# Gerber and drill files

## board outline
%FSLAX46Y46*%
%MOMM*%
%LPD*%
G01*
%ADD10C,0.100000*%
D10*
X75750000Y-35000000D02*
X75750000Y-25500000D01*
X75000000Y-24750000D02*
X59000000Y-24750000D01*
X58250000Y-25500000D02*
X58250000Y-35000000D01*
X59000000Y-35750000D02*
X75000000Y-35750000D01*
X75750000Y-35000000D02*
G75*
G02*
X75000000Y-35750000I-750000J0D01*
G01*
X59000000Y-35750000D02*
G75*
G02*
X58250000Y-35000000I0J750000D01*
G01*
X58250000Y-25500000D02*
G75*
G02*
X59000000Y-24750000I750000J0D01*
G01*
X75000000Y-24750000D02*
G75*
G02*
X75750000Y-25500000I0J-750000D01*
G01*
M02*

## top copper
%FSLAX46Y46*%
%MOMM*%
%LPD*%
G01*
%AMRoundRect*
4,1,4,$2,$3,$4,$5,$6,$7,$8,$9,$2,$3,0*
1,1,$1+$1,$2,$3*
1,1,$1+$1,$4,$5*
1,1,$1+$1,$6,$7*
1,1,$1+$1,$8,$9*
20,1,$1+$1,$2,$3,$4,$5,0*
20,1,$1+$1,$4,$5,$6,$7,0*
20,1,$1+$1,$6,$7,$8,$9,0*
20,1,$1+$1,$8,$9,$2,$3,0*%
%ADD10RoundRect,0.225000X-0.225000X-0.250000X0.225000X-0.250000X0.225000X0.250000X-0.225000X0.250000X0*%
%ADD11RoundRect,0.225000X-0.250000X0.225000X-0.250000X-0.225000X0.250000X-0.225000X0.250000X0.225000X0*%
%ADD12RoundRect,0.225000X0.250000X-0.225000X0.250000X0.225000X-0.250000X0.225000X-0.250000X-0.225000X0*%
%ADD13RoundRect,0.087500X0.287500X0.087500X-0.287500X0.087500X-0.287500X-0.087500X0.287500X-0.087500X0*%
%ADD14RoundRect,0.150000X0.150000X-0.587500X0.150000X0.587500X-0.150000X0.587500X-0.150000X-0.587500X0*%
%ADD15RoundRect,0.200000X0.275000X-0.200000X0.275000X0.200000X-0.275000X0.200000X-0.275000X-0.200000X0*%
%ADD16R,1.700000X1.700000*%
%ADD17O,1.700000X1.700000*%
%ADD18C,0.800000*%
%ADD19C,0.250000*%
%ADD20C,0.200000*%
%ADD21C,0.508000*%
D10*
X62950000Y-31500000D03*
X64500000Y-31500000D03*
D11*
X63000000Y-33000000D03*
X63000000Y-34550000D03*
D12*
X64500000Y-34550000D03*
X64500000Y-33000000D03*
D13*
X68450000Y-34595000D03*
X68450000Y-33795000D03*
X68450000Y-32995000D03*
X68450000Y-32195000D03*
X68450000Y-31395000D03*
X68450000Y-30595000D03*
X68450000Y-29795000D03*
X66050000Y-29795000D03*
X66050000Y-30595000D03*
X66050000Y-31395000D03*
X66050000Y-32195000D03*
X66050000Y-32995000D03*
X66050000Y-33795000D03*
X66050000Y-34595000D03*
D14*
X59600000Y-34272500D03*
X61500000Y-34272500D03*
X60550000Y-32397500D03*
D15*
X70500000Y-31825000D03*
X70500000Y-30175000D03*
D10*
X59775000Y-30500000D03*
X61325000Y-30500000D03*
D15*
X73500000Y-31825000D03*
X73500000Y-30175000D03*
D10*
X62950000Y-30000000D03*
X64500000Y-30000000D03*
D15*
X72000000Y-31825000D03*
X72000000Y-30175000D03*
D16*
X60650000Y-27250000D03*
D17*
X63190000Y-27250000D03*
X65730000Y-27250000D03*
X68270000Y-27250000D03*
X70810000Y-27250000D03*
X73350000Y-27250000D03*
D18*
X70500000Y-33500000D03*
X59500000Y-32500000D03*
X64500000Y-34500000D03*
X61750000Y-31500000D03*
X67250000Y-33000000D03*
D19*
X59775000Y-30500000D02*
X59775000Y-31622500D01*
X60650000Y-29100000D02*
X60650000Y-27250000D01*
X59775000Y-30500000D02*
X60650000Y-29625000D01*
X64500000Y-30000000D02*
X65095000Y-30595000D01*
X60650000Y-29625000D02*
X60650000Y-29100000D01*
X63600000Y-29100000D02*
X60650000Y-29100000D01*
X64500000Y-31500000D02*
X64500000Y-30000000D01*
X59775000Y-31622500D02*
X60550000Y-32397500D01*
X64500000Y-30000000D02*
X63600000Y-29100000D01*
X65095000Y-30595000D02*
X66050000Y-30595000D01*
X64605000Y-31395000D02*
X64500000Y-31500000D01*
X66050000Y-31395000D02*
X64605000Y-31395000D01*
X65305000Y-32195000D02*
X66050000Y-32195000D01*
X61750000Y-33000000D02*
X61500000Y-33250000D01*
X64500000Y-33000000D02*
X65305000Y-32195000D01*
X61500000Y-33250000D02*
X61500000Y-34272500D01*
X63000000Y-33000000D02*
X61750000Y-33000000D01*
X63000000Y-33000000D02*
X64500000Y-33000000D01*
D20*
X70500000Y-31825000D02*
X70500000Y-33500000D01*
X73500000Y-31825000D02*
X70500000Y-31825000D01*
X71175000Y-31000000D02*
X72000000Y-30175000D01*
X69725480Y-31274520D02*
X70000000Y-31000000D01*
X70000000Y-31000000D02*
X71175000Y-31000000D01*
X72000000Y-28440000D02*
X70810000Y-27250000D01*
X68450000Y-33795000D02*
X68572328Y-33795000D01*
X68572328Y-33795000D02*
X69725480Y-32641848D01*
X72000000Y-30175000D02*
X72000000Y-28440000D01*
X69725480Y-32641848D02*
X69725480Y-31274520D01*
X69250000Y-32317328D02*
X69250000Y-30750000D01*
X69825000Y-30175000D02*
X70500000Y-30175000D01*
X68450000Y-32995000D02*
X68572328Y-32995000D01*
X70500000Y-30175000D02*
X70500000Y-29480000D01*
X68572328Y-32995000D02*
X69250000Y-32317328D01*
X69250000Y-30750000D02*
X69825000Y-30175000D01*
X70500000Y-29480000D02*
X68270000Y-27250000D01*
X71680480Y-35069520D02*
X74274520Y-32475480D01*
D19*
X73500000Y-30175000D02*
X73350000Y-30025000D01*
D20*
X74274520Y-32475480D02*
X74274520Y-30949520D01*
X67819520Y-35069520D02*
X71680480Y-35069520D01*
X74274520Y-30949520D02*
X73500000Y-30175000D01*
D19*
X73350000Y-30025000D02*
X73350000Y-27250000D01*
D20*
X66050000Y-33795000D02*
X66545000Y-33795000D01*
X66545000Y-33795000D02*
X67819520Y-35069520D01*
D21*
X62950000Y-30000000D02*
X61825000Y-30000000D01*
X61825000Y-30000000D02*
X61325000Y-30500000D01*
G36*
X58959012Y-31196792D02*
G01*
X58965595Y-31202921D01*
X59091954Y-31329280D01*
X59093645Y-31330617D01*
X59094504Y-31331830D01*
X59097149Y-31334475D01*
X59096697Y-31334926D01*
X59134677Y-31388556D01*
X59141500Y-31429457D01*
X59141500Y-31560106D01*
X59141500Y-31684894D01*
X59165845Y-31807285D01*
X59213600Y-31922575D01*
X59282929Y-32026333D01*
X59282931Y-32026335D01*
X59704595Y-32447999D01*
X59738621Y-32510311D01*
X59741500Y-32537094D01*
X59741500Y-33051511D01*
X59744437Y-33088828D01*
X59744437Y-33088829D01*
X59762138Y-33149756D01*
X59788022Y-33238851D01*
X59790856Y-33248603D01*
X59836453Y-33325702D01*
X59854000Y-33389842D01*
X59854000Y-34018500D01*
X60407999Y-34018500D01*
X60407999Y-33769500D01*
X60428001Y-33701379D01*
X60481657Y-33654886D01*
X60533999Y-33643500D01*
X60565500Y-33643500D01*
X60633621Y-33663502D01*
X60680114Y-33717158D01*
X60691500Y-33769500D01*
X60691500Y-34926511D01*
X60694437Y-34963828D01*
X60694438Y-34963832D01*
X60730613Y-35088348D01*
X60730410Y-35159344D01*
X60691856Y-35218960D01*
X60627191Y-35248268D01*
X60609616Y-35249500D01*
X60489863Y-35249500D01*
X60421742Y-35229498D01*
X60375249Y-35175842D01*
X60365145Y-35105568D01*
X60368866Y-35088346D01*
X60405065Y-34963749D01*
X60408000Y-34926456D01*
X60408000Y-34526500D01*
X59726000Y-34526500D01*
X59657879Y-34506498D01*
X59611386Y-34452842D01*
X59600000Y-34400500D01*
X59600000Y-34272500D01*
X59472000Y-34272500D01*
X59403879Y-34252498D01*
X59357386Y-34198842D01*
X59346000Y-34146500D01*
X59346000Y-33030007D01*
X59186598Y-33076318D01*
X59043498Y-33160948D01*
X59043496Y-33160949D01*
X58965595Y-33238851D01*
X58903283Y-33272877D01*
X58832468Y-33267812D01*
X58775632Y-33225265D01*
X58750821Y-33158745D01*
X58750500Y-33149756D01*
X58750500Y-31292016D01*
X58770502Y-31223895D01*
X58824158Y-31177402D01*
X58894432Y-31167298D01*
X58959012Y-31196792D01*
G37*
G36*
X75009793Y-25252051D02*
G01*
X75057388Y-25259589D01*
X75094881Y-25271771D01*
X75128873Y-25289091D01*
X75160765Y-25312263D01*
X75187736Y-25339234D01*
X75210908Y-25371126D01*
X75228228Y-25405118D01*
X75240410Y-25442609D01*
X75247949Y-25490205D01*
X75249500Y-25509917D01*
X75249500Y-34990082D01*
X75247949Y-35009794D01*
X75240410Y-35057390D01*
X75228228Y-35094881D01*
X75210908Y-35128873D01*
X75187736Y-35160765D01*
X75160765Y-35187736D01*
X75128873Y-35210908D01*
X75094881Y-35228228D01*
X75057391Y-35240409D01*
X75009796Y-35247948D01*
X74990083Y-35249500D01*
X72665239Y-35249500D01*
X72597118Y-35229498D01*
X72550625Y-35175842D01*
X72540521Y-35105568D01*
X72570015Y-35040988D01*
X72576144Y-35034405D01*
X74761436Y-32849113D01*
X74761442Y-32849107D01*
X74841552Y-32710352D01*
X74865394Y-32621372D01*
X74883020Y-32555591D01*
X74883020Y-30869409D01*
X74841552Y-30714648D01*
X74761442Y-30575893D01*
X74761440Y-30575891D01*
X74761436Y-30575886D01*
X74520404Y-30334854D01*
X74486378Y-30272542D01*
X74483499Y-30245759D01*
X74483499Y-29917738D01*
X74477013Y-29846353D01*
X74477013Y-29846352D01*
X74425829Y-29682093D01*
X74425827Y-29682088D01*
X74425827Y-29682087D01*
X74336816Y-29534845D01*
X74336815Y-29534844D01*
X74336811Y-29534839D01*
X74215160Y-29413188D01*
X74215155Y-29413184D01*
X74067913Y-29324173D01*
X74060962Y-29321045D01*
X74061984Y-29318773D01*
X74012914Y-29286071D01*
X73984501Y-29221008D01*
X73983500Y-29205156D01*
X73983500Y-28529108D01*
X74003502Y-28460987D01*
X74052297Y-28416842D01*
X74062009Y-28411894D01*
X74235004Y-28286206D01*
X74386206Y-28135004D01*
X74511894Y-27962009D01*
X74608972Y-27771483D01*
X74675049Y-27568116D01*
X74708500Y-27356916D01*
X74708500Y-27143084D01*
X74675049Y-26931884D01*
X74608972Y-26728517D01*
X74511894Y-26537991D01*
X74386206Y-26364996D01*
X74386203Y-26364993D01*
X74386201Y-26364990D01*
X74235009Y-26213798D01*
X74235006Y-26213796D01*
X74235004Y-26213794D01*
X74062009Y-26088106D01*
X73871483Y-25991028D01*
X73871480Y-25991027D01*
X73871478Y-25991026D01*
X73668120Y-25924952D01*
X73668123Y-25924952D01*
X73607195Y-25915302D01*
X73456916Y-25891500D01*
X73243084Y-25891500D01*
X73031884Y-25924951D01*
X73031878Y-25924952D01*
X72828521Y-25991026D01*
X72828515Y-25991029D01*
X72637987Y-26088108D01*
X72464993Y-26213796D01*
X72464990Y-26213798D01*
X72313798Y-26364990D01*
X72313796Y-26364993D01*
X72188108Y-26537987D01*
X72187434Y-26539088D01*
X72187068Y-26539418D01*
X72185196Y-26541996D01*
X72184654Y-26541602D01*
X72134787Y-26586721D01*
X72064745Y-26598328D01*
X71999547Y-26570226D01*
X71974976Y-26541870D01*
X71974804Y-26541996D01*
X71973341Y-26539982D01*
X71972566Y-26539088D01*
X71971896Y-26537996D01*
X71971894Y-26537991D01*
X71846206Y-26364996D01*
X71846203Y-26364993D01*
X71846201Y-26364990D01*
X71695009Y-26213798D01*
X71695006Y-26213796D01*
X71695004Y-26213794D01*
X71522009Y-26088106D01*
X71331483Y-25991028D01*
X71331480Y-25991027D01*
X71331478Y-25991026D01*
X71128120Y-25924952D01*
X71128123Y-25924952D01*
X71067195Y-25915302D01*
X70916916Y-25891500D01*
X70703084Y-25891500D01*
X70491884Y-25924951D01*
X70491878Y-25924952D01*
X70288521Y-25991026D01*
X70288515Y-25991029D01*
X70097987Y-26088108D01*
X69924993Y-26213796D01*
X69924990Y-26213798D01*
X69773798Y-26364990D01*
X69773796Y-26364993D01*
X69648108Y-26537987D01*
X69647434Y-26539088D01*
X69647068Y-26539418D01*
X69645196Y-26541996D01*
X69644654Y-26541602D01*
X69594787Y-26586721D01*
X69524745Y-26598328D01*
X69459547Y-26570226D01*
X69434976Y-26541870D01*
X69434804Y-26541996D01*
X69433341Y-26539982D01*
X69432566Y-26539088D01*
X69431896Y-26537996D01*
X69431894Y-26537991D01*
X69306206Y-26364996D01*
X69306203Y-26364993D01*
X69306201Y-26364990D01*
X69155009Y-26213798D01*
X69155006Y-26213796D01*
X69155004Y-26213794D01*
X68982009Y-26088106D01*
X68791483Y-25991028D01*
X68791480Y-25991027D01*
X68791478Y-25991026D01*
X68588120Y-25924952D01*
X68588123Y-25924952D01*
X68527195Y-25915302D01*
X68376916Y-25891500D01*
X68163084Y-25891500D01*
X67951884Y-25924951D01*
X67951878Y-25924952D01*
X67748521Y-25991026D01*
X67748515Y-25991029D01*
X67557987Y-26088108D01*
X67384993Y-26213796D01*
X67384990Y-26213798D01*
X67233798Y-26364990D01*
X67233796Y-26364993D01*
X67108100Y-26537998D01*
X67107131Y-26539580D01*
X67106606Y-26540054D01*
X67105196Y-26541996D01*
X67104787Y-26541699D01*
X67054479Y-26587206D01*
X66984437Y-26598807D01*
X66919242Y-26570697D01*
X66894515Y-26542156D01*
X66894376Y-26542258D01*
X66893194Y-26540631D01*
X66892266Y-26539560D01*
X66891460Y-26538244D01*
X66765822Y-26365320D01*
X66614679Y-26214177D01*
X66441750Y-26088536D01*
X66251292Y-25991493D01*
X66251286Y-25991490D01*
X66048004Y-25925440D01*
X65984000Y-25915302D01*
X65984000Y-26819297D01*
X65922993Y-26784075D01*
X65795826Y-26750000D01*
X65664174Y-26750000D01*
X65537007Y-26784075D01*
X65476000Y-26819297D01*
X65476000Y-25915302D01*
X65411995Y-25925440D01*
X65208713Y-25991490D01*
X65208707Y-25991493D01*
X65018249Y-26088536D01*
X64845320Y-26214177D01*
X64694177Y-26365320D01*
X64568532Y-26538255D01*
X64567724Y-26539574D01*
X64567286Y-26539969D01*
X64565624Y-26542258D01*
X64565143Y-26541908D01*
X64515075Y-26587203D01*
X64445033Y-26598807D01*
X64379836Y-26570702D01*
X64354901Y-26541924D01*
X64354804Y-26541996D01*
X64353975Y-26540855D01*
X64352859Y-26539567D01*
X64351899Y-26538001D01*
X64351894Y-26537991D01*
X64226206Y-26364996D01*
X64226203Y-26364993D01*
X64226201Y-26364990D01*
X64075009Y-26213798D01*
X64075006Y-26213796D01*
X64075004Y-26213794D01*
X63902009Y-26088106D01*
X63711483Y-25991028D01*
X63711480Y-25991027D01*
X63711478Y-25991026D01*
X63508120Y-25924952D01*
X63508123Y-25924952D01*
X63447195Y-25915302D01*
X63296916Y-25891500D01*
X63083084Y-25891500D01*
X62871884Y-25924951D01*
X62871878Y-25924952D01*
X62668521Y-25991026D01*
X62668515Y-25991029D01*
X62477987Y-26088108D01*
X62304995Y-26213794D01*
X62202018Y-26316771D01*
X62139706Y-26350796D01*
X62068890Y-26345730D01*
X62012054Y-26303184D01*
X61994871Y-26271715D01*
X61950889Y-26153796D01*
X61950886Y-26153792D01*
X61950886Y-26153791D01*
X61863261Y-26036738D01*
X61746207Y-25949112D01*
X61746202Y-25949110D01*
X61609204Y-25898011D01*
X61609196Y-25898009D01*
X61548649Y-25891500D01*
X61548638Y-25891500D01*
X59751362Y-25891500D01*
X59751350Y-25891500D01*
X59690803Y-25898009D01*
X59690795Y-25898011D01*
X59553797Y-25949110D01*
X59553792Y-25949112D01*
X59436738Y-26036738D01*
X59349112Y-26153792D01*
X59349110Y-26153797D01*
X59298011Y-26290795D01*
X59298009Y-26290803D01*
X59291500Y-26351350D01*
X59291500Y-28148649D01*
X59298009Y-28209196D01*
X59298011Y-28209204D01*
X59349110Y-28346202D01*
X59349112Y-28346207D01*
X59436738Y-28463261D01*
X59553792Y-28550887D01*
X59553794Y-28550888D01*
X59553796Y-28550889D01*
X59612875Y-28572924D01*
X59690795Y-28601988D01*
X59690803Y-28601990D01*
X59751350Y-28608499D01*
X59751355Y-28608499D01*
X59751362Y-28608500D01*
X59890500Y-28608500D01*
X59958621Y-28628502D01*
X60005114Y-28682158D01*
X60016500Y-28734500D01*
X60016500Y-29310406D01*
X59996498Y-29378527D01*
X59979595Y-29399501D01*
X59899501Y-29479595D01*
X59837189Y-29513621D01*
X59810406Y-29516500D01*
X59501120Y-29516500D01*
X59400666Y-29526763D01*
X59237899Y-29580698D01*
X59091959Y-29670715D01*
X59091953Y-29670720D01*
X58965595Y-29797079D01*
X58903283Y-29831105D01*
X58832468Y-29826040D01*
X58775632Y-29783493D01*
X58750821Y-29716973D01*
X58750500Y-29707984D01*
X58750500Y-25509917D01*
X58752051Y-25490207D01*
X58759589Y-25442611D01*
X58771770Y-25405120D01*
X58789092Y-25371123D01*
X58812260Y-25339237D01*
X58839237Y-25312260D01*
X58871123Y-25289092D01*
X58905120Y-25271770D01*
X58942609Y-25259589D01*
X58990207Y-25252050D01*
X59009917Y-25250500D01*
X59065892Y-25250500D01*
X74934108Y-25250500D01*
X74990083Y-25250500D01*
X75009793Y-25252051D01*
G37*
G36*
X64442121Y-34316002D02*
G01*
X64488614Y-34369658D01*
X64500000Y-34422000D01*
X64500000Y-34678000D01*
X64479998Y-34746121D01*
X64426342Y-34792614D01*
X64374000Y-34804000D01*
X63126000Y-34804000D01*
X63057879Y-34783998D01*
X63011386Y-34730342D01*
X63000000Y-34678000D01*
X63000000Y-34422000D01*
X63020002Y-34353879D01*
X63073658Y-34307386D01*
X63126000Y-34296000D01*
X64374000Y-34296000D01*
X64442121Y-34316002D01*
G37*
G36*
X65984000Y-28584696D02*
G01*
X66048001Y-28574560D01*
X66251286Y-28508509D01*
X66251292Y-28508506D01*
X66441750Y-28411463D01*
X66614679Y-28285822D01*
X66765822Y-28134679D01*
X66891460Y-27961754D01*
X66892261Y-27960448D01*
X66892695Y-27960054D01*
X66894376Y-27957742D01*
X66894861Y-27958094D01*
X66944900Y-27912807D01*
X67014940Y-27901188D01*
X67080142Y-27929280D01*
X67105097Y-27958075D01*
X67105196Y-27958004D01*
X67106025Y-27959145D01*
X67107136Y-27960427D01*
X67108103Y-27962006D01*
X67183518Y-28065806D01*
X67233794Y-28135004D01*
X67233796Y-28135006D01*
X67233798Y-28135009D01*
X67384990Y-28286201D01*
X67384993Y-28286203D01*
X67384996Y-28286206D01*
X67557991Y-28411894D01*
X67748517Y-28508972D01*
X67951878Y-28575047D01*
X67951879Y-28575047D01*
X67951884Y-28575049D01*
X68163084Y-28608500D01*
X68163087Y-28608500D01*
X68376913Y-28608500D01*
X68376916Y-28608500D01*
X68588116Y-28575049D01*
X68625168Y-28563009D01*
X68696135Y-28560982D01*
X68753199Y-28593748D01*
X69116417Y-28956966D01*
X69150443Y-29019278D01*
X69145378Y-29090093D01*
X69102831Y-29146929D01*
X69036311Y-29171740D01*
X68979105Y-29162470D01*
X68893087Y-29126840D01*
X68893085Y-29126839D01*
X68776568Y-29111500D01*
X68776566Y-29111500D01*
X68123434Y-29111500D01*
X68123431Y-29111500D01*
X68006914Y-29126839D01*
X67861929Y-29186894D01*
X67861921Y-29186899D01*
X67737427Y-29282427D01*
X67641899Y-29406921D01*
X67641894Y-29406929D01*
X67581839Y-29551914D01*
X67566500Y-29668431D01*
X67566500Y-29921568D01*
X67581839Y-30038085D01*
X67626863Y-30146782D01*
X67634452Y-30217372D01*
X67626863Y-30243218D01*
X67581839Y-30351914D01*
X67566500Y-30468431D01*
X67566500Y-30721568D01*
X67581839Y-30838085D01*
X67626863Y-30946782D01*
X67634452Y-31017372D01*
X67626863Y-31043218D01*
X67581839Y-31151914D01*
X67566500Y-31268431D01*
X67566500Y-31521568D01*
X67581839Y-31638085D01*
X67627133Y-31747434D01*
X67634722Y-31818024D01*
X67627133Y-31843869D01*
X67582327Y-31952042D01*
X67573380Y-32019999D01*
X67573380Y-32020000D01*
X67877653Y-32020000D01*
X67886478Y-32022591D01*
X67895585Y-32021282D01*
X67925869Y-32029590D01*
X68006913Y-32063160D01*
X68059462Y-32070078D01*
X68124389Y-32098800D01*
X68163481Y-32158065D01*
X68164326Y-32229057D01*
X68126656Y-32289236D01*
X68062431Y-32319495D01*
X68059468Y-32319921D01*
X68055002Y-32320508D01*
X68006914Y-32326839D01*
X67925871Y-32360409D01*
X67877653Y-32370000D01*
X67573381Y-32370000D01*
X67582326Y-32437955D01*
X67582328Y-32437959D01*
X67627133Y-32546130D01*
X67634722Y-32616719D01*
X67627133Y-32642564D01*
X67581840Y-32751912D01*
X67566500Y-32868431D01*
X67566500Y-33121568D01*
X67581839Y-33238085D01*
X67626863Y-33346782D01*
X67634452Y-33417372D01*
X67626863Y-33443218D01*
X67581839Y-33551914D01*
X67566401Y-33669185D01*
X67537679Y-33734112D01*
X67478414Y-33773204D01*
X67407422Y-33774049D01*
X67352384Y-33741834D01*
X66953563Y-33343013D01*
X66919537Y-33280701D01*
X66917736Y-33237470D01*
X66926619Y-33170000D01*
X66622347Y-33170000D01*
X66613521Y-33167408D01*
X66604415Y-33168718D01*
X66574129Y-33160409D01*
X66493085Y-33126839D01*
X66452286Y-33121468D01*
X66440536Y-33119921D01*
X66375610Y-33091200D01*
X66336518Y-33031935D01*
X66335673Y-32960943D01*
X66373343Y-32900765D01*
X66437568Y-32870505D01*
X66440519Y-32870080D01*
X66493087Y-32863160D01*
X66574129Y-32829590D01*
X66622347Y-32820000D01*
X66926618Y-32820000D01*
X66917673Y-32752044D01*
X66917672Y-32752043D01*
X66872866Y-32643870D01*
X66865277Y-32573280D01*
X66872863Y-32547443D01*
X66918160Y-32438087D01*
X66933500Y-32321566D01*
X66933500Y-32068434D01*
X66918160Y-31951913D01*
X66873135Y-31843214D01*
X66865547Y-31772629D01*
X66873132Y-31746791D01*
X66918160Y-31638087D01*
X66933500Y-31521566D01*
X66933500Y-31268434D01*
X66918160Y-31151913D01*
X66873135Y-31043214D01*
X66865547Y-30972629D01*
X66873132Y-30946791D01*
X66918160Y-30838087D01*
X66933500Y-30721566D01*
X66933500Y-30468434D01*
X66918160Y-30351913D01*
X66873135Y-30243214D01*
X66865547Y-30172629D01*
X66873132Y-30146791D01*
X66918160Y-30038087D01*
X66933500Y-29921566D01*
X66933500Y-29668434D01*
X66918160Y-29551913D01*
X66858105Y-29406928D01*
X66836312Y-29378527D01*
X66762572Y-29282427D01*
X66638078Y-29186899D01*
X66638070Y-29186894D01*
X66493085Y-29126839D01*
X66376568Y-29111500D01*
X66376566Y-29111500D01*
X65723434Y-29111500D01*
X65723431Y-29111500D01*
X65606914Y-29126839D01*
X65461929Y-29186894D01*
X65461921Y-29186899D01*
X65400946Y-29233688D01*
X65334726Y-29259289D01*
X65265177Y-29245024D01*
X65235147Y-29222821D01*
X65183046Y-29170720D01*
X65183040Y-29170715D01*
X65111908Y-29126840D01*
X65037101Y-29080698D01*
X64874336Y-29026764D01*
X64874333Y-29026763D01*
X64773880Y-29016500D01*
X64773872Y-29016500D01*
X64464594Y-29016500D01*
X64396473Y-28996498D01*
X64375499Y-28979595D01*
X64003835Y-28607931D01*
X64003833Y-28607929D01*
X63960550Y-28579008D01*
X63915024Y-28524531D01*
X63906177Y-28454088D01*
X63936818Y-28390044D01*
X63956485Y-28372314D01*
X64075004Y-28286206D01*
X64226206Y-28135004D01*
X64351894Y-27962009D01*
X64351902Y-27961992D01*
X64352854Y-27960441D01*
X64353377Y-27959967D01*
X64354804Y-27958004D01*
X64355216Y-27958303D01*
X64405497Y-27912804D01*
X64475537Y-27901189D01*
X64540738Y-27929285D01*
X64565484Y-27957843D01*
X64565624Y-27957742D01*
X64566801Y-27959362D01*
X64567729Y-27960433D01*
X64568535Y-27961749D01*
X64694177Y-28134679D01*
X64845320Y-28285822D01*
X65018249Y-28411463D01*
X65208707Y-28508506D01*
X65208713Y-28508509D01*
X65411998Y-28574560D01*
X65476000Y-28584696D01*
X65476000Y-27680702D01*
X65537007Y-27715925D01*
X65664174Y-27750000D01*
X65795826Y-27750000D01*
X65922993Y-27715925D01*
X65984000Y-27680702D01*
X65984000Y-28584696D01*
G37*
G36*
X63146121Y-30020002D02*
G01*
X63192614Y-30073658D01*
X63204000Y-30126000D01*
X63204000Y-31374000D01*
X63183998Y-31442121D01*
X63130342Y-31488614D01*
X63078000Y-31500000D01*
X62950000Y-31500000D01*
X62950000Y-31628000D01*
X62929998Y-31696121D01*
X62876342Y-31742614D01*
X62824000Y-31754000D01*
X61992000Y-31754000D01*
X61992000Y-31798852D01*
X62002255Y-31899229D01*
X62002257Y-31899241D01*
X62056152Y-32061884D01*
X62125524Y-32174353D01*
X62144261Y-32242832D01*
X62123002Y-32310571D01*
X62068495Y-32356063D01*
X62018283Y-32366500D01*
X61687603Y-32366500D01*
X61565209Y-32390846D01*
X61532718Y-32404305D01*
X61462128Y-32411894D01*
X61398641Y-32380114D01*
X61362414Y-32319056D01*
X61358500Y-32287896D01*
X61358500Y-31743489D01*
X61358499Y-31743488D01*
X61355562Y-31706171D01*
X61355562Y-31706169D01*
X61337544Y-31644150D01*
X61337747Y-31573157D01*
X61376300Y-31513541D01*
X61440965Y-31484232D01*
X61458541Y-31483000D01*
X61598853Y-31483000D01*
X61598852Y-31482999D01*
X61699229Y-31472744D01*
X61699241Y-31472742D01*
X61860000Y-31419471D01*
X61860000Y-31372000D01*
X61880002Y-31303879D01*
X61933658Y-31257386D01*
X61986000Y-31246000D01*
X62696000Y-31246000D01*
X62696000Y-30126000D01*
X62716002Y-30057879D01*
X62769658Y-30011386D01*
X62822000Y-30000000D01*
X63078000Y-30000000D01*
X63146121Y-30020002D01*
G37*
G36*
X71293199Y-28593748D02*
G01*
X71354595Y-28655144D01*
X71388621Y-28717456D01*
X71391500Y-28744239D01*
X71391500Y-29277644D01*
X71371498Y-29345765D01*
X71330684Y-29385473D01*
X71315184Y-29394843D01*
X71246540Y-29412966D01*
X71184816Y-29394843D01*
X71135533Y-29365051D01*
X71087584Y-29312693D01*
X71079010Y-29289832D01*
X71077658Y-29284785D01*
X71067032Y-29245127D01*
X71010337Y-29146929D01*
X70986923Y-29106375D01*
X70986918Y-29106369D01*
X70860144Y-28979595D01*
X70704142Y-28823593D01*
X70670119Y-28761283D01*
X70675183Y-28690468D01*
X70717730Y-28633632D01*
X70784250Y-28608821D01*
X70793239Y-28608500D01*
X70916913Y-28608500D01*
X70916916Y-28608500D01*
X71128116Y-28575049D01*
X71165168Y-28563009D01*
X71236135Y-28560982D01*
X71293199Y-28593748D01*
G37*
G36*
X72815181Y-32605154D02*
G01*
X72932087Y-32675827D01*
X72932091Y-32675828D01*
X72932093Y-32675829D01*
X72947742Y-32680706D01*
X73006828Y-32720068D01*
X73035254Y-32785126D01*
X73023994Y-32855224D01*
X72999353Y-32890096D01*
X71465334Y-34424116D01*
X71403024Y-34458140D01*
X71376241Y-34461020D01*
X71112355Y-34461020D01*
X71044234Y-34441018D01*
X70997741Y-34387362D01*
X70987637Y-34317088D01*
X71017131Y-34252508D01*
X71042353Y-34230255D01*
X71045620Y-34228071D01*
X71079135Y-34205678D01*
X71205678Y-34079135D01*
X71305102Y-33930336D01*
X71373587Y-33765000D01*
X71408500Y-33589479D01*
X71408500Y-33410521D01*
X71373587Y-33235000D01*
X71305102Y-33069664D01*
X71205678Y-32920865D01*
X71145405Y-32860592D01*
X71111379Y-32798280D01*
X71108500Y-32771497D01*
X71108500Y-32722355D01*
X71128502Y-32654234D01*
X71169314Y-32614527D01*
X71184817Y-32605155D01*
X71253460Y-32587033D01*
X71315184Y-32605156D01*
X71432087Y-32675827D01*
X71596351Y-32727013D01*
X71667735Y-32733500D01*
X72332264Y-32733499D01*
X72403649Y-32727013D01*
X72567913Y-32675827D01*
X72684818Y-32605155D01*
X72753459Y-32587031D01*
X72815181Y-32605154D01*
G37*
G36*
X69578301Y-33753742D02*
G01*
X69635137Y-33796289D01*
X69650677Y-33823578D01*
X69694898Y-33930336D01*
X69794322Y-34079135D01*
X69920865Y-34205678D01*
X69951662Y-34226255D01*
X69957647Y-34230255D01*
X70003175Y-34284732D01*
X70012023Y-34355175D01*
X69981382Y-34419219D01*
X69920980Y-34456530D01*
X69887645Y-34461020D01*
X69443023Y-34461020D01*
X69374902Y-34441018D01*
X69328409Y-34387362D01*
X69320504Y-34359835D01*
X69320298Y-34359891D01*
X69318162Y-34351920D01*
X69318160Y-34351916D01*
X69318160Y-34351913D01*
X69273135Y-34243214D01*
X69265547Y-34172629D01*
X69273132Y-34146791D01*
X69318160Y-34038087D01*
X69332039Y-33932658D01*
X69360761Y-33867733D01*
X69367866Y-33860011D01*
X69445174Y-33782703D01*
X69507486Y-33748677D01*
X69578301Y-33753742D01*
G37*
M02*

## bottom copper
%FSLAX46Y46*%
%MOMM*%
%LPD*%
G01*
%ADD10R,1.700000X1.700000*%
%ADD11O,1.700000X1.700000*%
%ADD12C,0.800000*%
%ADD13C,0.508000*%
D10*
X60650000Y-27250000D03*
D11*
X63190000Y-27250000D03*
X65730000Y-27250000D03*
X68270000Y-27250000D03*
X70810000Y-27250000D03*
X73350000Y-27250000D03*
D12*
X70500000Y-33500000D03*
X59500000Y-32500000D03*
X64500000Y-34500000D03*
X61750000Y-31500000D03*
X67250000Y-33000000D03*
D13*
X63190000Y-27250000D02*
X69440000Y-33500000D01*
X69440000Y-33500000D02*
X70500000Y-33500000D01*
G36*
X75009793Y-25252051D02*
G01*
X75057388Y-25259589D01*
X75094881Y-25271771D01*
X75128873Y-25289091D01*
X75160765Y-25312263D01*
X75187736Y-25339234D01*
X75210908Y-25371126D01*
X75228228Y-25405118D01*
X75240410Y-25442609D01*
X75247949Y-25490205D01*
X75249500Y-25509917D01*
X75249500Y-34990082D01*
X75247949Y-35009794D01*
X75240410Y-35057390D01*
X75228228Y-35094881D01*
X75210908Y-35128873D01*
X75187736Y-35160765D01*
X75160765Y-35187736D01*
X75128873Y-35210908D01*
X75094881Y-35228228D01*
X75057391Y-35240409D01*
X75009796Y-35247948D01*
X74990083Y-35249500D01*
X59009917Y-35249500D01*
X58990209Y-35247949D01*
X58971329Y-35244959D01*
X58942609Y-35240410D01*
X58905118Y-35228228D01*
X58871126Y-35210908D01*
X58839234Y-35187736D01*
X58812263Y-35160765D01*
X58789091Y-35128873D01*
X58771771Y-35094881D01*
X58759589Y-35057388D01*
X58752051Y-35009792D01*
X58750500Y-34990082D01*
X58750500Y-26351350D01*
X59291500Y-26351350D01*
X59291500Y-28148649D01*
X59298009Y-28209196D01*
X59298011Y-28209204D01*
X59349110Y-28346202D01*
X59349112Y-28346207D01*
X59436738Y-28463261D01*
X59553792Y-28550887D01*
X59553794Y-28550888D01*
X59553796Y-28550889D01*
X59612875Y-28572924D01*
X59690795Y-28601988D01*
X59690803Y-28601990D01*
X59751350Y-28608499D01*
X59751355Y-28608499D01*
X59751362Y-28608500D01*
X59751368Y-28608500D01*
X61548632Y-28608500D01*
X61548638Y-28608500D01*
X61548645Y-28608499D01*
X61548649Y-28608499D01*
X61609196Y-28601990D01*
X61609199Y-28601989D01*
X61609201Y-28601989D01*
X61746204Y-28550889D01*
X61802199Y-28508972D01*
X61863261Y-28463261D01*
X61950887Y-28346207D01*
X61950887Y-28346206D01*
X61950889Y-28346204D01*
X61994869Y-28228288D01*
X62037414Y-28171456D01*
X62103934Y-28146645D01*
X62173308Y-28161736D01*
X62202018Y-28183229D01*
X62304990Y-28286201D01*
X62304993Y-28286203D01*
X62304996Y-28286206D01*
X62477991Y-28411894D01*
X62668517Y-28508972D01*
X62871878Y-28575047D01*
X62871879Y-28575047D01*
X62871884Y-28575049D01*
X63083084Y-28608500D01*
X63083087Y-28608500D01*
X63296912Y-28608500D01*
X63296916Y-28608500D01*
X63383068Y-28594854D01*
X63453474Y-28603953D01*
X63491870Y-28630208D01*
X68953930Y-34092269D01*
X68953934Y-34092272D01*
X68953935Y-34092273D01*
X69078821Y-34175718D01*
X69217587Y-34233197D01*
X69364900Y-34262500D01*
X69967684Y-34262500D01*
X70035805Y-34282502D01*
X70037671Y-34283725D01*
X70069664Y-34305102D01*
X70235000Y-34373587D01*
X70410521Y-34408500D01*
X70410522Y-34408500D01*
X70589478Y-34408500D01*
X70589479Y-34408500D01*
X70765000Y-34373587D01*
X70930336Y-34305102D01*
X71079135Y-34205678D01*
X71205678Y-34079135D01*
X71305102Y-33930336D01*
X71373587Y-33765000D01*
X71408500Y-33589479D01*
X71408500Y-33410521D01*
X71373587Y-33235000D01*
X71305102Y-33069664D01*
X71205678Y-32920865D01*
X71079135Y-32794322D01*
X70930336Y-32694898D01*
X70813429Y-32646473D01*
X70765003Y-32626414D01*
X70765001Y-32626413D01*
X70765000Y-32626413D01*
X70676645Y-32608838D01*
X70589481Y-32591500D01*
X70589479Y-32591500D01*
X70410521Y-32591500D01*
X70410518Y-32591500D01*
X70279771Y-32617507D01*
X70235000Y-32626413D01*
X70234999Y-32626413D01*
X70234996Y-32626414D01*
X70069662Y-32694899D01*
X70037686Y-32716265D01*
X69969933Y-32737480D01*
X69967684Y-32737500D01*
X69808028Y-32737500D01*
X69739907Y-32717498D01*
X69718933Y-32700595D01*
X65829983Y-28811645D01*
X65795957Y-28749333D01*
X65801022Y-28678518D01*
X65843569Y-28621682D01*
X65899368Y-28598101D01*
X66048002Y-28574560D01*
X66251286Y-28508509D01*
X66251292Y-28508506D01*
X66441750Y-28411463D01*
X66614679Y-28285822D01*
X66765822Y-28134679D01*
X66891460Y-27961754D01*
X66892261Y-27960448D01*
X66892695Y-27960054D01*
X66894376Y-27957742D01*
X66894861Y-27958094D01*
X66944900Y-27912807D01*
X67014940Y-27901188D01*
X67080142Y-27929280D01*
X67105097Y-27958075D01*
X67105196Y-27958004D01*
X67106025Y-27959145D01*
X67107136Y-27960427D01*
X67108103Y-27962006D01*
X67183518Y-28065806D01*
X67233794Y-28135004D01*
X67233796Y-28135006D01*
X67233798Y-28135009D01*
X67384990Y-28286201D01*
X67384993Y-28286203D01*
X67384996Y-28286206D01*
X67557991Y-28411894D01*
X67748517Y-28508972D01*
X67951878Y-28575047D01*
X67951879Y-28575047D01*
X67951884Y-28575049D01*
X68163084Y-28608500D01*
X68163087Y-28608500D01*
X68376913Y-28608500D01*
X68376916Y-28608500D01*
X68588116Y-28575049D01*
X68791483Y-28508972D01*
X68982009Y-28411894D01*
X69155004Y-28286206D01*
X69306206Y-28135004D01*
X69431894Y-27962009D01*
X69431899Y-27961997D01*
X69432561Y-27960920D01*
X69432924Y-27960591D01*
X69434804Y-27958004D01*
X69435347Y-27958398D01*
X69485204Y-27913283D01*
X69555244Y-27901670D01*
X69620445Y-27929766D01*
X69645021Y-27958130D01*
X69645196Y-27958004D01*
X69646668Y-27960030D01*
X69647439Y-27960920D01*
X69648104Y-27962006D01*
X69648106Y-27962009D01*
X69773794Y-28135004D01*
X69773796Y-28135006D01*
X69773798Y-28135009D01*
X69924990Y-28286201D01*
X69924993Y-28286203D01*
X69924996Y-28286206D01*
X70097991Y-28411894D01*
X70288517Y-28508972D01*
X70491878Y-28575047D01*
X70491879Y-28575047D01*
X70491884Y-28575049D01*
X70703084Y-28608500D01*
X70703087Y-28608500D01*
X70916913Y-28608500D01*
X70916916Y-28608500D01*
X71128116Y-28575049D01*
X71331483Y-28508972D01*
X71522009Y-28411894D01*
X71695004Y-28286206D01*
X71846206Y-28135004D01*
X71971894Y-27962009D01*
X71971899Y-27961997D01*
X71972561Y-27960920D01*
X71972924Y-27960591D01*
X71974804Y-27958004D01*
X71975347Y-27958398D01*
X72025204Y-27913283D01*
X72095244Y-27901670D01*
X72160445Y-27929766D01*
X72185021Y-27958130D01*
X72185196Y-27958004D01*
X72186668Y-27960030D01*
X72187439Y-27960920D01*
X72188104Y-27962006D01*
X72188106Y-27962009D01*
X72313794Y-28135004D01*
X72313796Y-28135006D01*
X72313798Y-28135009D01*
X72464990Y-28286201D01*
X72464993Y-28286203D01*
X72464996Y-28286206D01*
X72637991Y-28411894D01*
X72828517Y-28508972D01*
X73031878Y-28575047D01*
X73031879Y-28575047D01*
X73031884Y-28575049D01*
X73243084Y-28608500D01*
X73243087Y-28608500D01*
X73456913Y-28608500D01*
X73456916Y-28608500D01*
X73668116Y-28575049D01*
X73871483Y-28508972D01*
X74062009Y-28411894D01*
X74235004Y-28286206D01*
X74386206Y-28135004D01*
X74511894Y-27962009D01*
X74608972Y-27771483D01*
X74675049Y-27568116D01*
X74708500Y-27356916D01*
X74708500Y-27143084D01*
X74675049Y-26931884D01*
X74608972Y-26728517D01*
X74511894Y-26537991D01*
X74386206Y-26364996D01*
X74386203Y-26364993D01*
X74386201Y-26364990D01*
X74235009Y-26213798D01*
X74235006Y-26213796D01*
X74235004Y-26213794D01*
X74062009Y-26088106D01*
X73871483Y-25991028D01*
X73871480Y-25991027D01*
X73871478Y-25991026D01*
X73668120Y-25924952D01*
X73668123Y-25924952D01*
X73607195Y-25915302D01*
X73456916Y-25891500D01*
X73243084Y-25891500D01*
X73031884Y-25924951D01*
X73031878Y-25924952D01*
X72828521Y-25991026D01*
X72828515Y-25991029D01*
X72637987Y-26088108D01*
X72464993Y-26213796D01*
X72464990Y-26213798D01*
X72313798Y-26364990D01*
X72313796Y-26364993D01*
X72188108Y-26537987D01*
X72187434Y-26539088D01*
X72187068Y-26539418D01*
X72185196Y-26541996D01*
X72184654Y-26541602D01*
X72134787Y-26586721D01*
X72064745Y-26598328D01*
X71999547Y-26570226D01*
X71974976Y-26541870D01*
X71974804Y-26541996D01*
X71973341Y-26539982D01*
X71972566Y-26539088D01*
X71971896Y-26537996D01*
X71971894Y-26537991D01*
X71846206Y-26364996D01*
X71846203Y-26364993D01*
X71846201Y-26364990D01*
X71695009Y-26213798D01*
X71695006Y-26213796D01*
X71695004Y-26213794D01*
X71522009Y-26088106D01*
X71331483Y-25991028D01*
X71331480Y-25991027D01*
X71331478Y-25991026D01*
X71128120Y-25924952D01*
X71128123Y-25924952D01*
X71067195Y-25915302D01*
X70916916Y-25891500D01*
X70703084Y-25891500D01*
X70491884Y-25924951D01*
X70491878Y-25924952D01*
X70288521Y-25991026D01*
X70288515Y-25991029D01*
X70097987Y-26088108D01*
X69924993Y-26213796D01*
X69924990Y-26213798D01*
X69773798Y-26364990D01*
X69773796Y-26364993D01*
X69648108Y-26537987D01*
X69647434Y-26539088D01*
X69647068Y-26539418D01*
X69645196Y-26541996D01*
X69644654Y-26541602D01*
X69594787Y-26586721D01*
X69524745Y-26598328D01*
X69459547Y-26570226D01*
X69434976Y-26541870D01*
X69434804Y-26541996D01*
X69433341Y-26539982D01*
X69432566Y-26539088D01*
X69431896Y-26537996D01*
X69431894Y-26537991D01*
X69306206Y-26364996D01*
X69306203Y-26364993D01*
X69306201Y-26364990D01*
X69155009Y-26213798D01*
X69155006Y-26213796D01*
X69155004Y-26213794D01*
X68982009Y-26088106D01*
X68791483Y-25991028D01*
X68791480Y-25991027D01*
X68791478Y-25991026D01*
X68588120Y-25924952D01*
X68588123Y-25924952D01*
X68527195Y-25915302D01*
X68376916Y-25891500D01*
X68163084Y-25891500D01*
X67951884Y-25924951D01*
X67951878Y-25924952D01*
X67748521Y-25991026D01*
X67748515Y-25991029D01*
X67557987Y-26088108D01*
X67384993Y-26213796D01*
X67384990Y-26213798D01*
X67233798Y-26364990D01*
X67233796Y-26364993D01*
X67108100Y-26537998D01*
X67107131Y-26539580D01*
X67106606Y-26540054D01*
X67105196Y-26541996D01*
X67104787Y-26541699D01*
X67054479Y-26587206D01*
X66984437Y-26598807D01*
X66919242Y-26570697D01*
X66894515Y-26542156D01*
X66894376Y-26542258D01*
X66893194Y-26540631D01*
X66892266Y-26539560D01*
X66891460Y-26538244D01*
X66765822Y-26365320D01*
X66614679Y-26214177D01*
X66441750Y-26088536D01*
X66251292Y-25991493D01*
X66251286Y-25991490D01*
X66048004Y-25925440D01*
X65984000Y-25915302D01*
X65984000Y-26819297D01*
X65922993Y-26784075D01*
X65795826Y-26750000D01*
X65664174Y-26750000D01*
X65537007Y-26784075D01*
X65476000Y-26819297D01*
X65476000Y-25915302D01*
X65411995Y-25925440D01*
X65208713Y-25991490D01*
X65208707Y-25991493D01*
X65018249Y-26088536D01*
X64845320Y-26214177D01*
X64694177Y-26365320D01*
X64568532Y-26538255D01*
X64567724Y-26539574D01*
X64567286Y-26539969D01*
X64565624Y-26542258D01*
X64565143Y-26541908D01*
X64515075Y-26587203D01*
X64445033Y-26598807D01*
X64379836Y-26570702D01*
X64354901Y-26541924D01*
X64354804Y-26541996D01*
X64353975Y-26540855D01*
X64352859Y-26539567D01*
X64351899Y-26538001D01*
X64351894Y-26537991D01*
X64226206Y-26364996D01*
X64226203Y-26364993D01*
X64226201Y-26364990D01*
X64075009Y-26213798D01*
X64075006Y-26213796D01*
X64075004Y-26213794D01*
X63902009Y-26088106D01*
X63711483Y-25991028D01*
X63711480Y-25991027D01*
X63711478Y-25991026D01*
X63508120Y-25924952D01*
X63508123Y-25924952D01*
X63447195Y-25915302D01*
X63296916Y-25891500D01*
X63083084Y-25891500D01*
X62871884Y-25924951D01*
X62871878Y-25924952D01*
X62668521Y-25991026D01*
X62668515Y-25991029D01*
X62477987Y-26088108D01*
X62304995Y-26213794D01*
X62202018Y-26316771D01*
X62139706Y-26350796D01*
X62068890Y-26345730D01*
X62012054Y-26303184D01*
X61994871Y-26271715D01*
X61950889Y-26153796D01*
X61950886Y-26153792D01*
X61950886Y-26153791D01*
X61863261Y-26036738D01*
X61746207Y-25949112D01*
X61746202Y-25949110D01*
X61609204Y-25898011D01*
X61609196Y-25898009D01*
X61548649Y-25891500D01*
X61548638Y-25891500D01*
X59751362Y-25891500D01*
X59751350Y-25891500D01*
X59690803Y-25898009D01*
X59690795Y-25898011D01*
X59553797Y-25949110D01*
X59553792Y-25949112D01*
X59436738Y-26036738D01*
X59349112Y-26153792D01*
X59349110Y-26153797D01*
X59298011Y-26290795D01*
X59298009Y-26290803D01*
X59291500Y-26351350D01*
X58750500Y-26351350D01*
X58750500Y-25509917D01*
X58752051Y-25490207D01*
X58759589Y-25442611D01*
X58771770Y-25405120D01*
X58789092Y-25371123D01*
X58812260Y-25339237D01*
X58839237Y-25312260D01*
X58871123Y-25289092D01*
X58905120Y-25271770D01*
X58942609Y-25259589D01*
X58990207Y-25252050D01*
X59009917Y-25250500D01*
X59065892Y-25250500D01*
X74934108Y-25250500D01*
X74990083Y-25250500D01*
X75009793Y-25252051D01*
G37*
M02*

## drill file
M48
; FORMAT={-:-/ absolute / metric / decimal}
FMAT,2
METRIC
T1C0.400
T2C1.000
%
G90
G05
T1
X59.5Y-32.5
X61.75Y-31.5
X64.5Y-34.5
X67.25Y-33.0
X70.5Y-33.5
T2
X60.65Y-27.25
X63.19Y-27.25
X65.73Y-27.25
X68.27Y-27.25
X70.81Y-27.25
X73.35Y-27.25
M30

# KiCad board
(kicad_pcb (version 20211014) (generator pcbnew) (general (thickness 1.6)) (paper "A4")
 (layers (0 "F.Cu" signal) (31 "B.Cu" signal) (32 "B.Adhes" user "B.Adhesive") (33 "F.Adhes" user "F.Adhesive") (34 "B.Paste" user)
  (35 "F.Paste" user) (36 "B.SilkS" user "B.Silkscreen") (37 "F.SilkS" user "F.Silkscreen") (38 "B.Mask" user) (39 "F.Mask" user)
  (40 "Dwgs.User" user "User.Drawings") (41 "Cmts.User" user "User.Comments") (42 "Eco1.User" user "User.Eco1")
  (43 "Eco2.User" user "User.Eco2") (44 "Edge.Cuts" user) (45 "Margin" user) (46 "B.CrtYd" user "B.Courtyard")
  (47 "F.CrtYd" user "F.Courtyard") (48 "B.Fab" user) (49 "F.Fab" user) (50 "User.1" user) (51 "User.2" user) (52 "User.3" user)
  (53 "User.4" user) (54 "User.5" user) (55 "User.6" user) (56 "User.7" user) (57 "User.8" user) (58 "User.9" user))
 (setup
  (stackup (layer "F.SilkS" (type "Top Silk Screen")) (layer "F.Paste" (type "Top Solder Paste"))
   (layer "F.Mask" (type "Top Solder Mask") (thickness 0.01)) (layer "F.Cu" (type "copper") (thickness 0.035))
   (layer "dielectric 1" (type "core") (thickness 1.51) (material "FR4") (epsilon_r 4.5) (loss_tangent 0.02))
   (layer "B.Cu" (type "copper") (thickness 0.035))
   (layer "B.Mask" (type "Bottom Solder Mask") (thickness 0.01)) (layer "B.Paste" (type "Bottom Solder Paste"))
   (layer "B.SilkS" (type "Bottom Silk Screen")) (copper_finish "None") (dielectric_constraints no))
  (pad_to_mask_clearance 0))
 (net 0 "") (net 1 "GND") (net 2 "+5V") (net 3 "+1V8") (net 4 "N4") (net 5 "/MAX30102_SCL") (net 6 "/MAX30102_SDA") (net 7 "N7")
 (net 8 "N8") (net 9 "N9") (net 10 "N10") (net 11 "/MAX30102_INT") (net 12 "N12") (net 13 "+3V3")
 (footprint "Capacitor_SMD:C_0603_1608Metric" (layer "F.Cu") (at 63.725 31.5)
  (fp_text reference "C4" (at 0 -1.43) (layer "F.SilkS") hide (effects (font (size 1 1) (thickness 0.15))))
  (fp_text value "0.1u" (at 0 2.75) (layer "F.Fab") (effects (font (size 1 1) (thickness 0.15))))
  (pad "1" smd roundrect (at -0.775 0) (size 0.9 0.95) (layers "F.Cu" "F.Paste" "F.Mask") (roundrect_rratio 0.25) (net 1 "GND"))
  (pad "2" smd roundrect (at 0.775 0) (size 0.9 0.95) (layers "F.Cu" "F.Paste" "F.Mask") (roundrect_rratio 0.25) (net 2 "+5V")))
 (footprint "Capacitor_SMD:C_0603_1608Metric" (layer "F.Cu") (at 63 33.775 -90)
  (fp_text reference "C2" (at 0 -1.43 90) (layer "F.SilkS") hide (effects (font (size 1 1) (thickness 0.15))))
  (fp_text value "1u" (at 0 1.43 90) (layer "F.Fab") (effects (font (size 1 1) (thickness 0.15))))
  (pad "1" smd roundrect (at -0.775 0 270) (size 0.9 0.95) (layers "F.Cu" "F.Paste" "F.Mask") (roundrect_rratio 0.25) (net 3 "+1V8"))
  (pad "2" smd roundrect (at 0.775 0 270) (size 0.9 0.95) (layers "F.Cu" "F.Paste" "F.Mask") (roundrect_rratio 0.25) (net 1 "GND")))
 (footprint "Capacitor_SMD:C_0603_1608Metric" (layer "F.Cu") (at 64.5 33.775 90)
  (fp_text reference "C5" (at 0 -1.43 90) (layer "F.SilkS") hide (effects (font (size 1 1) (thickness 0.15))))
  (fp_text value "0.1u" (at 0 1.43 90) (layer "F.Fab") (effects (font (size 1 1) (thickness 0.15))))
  (pad "1" smd roundrect (at -0.775 0 90) (size 0.9 0.95) (layers "F.Cu" "F.Paste" "F.Mask") (roundrect_rratio 0.25) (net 1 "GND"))
  (pad "2" smd roundrect (at 0.775 0 90) (size 0.9 0.95) (layers "F.Cu" "F.Paste" "F.Mask") (roundrect_rratio 0.25) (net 3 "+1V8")))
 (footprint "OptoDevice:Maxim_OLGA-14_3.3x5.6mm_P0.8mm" (layer "F.Cu") (at 67.25 32.195 180)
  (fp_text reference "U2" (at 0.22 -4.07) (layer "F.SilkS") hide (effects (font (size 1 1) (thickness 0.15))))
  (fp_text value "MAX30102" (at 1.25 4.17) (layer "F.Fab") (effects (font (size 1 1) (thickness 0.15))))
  (pad "1" smd roundrect (at -1.2 -2.4 180) (size 0.75 0.35) (layers "F.Cu" "F.Paste" "F.Mask") (roundrect_rratio 0.25) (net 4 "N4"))
  (pad "2" smd roundrect (at -1.2 -1.6 180) (size 0.75 0.35) (layers "F.Cu" "F.Paste" "F.Mask") (roundrect_rratio 0.25)
   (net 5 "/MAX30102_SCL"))
  (pad "3" smd roundrect (at -1.2 -0.8 180) (size 0.75 0.35) (layers "F.Cu" "F.Paste" "F.Mask") (roundrect_rratio 0.25)
   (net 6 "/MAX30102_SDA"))
  (pad "4" smd roundrect (at -1.2 0 180) (size 0.75 0.35) (layers "F.Cu" "F.Paste" "F.Mask") (roundrect_rratio 0.25) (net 1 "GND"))
  (pad "5" smd roundrect (at -1.2 0.8 180) (size 0.75 0.35) (layers "F.Cu" "F.Paste" "F.Mask") (roundrect_rratio 0.25) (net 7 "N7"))
  (pad "6" smd roundrect (at -1.2 1.6 180) (size 0.75 0.35) (layers "F.Cu" "F.Paste" "F.Mask") (roundrect_rratio 0.25) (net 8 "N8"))
  (pad "7" smd roundrect (at -1.2 2.4 180) (size 0.75 0.35) (layers "F.Cu" "F.Paste" "F.Mask") (roundrect_rratio 0.25) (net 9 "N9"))
  (pad "8" smd roundrect (at 1.2 2.4 180) (size 0.75 0.35) (layers "F.Cu" "F.Paste" "F.Mask") (roundrect_rratio 0.25) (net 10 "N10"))
  (pad "9" smd roundrect (at 1.2 1.6 180) (size 0.75 0.35) (layers "F.Cu" "F.Paste" "F.Mask") (roundrect_rratio 0.25) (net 2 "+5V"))
  (pad "10" smd roundrect (at 1.2 0.8 180) (size 0.75 0.35) (layers "F.Cu" "F.Paste" "F.Mask") (roundrect_rratio 0.25) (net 2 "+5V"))
  (pad "11" smd roundrect (at 1.2 0 180) (size 0.75 0.35) (layers "F.Cu" "F.Paste" "F.Mask") (roundrect_rratio 0.25) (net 3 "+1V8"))
  (pad "12" smd roundrect (at 1.2 -0.8 180) (size 0.75 0.35) (layers "F.Cu" "F.Paste" "F.Mask") (roundrect_rratio 0.25) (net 1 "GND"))
  (pad "13" smd roundrect (at 1.2 -1.6 180) (size 0.75 0.35) (layers "F.Cu" "F.Paste" "F.Mask") (roundrect_rratio 0.25)
   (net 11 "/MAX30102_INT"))
  (pad "14" smd roundrect (at 1.2 -2.4 180) (size 0.75 0.35) (layers "F.Cu" "F.Paste" "F.Mask") (roundrect_rratio 0.25) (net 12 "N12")))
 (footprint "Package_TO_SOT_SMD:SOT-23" (layer "F.Cu") (at 60.55 33.335 90)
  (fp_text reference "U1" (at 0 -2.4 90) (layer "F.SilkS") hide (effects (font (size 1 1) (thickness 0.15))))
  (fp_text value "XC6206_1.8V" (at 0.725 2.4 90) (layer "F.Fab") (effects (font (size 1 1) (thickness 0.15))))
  (pad "1" smd roundrect (at -0.9375 -0.95 90) (size 1.475 0.6) (layers "F.Cu" "F.Paste" "F.Mask") (roundrect_rratio 0.25) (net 1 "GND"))
  (pad "2" smd roundrect (at -0.9375 0.95 90) (size 1.475 0.6) (layers "F.Cu" "F.Paste" "F.Mask") (roundrect_rratio 0.25) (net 3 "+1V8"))
  (pad "3" smd roundrect (at 0.9375 0 90) (size 1.475 0.6) (layers "F.Cu" "F.Paste" "F.Mask") (roundrect_rratio 0.25) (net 2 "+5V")))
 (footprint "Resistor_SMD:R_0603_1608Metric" (layer "F.Cu") (at 70.5 31 90)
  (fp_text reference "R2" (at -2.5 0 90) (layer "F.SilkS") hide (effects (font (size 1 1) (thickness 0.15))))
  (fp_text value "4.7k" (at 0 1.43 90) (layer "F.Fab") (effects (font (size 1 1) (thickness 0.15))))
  (pad "1" smd roundrect (at -0.825 0 90) (size 0.8 0.95) (layers "F.Cu" "F.Paste" "F.Mask") (roundrect_rratio 0.25) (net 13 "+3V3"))
  (pad "2" smd roundrect (at 0.825 0 90) (size 0.8 0.95) (layers "F.Cu" "F.Paste" "F.Mask") (roundrect_rratio 0.25) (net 6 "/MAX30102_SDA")))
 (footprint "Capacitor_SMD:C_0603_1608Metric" (layer "F.Cu") (at 60.55 30.5)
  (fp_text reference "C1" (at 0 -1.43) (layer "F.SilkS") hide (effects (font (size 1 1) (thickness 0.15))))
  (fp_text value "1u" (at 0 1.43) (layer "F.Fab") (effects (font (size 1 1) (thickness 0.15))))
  (pad "1" smd roundrect (at -0.775 0) (size 0.9 0.95) (layers "F.Cu" "F.Paste" "F.Mask") (roundrect_rratio 0.25) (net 2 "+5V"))
  (pad "2" smd roundrect (at 0.775 0) (size 0.9 0.95) (layers "F.Cu" "F.Paste" "F.Mask") (roundrect_rratio 0.25) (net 1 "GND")))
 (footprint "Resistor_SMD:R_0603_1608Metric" (layer "F.Cu") (at 73.5 31 90)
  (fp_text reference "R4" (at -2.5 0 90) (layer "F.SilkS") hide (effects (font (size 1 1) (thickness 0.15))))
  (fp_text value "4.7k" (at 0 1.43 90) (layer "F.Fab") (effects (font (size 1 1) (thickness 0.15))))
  (pad "1" smd roundrect (at -0.825 0 90) (size 0.8 0.95) (layers "F.Cu" "F.Paste" "F.Mask") (roundrect_rratio 0.25) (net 13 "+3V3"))
  (pad "2" smd roundrect (at 0.825 0 90) (size 0.8 0.95) (layers "F.Cu" "F.Paste" "F.Mask") (roundrect_rratio 0.25) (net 11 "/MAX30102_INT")))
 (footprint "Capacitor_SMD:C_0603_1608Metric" (layer "F.Cu") (at 63.725 30)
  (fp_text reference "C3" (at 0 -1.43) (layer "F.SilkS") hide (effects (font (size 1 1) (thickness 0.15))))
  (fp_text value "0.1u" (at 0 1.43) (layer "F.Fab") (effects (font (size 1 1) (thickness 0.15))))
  (pad "1" smd roundrect (at -0.775 0) (size 0.9 0.95) (layers "F.Cu" "F.Paste" "F.Mask") (roundrect_rratio 0.25) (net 1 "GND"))
  (pad "2" smd roundrect (at 0.775 0) (size 0.9 0.95) (layers "F.Cu" "F.Paste" "F.Mask") (roundrect_rratio 0.25) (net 2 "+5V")))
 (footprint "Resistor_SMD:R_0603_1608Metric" (layer "F.Cu") (at 72 31 90)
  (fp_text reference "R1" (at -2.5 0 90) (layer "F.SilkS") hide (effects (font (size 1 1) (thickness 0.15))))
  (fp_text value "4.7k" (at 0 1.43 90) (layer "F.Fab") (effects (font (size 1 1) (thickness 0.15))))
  (pad "1" smd roundrect (at -0.825 0 90) (size 0.8 0.95) (layers "F.Cu" "F.Paste" "F.Mask") (roundrect_rratio 0.25) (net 13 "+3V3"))
  (pad "2" smd roundrect (at 0.825 0 90) (size 0.8 0.95) (layers "F.Cu" "F.Paste" "F.Mask") (roundrect_rratio 0.25) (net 5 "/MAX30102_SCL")))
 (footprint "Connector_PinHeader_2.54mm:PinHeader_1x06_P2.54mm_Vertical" (layer "F.Cu") (at 60.65 27.25 90)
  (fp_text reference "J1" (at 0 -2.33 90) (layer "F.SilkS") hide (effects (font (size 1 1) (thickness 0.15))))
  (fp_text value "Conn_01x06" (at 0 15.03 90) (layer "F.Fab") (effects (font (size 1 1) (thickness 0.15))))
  (pad "1" thru_hole rect (at 0 0 90) (size 1.7 1.7) (drill 1) (layers *.Cu *.Mask) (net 2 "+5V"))
  (pad "2" thru_hole oval (at 0 2.54 90) (size 1.7 1.7) (drill 1) (layers *.Cu *.Mask) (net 13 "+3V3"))
  (pad "3" thru_hole oval (at 0 5.08 90) (size 1.7 1.7) (drill 1) (layers *.Cu *.Mask) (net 1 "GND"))
  (pad "4" thru_hole oval (at 0 7.62 90) (size 1.7 1.7) (drill 1) (layers *.Cu *.Mask) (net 6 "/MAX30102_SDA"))
  (pad "5" thru_hole oval (at 0 10.16 90) (size 1.7 1.7) (drill 1) (layers *.Cu *.Mask) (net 5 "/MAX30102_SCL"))
  (pad "6" thru_hole oval (at 0 12.7 90) (size 1.7 1.7) (drill 1) (layers *.Cu *.Mask) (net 11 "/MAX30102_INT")))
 (gr_line (start 75.75 35) (end 75.75 25.5) (layer "Edge.Cuts") (width 0.1))
 (gr_line (start 75 24.75) (end 59 24.75) (layer "Edge.Cuts") (width 0.1))
 (gr_line (start 58.25 25.5) (end 58.25 35) (layer "Edge.Cuts") (width 0.1))
 (gr_line (start 59 35.75) (end 75 35.75) (layer "Edge.Cuts") (width 0.1))
 (gr_arc (start 75.75 35) (mid 75.53033 35.53033) (end 75 35.75) (layer "Edge.Cuts") (width 0.1))
 (gr_arc (start 59 35.75) (mid 58.46967 35.53033) (end 58.25 35) (layer "Edge.Cuts") (width 0.1))
 (gr_arc (start 58.25 25.5) (mid 58.46967 24.96967) (end 59 24.75) (layer "Edge.Cuts") (width 0.1))
 (gr_arc (start 75 24.75) (mid 75.53033 24.96967) (end 75.75 25.5) (layer "Edge.Cuts") (width 0.1))
 (segment (start 59.775 30.5) (end 59.775 31.6225) (width 0.25) (layer "F.Cu") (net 2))
 (segment (start 60.65 29.1) (end 60.65 27.25) (width 0.25) (layer "F.Cu") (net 2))
 (segment (start 59.775 30.5) (end 60.65 29.625) (width 0.25) (layer "F.Cu") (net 2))
 (segment (start 64.5 30) (end 65.095 30.595) (width 0.25) (layer "F.Cu") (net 2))
 (segment (start 60.65 29.625) (end 60.65 29.1) (width 0.25) (layer "F.Cu") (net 2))
 (segment (start 63.6 29.1) (end 60.65 29.1) (width 0.25) (layer "F.Cu") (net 2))
 (segment (start 64.5 31.5) (end 64.5 30) (width 0.25) (layer "F.Cu") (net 2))
 (segment (start 59.775 31.6225) (end 60.55 32.3975) (width 0.25) (layer "F.Cu") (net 2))
 (segment (start 64.5 30) (end 63.6 29.1) (width 0.25) (layer "F.Cu") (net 2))
 (segment (start 65.095 30.595) (end 66.05 30.595) (width 0.25) (layer "F.Cu") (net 2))
 (segment (start 64.605 31.395) (end 64.5 31.5) (width 0.25) (layer "F.Cu") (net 2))
 (segment (start 66.05 31.395) (end 64.605 31.395) (width 0.25) (layer "F.Cu") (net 2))
 (segment (start 65.305 32.195) (end 66.05 32.195) (width 0.25) (layer "F.Cu") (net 3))
 (segment (start 61.75 33) (end 61.5 33.25) (width 0.25) (layer "F.Cu") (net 3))
 (segment (start 64.5 33) (end 65.305 32.195) (width 0.25) (layer "F.Cu") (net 3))
 (segment (start 61.5 33.25) (end 61.5 34.2725) (width 0.25) (layer "F.Cu") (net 3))
 (segment (start 63 33) (end 61.75 33) (width 0.25) (layer "F.Cu") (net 3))
 (segment (start 63 33) (end 64.5 33) (width 0.25) (layer "F.Cu") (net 3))
 (segment (start 70.5 31.825) (end 70.5 33.5) (width 0.2) (layer "F.Cu") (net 13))
 (segment (start 73.5 31.825) (end 70.5 31.825) (width 0.2) (layer "F.Cu") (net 13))
 (via (at 70.5 33.5) (size 0.8) (drill 0.4) (layers "F.Cu" "B.Cu") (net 13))
 (segment (start 63.19 27.25) (end 69.44 33.5) (width 0.508) (layer "B.Cu") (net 13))
 (segment (start 69.44 33.5) (end 70.5 33.5) (width 0.508) (layer "B.Cu") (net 13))
 (segment (start 71.175 31) (end 72 30.175) (width 0.2) (layer "F.Cu") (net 5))
 (segment (start 69.72548 31.27452) (end 70 31) (width 0.2) (layer "F.Cu") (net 5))
 (segment (start 70 31) (end 71.175 31) (width 0.2) (layer "F.Cu") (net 5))
 (segment (start 72 28.44) (end 70.81 27.25) (width 0.2) (layer "F.Cu") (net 5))
 (segment (start 68.45 33.795) (end 68.572328 33.795) (width 0.2) (layer "F.Cu") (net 5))
 (segment (start 68.572328 33.795) (end 69.72548 32.641848) (width 0.2) (layer "F.Cu") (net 5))
 (segment (start 72 30.175) (end 72 28.44) (width 0.2) (layer "F.Cu") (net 5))
 (segment (start 69.72548 32.641848) (end 69.72548 31.27452) (width 0.2) (layer "F.Cu") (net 5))
 (segment (start 69.25 32.317328) (end 69.25 30.75) (width 0.2) (layer "F.Cu") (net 6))
 (segment (start 69.825 30.175) (end 70.5 30.175) (width 0.2) (layer "F.Cu") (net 6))
 (segment (start 68.45 32.995) (end 68.572328 32.995) (width 0.2) (layer "F.Cu") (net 6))
 (segment (start 70.5 30.175) (end 70.5 29.48) (width 0.2) (layer "F.Cu") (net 6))
 (segment (start 68.572328 32.995) (end 69.25 32.317328) (width 0.2) (layer "F.Cu") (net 6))
 (segment (start 69.25 30.75) (end 69.825 30.175) (width 0.2) (layer "F.Cu") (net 6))
 (segment (start 70.5 29.48) (end 68.27 27.25) (width 0.2) (layer "F.Cu") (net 6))
 (segment (start 71.68048 35.06952) (end 74.27452 32.47548) (width 0.2) (layer "F.Cu") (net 11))
 (segment (start 73.5 30.175) (end 73.35 30.025) (width 0.25) (layer "F.Cu") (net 11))
 (segment (start 74.27452 32.47548) (end 74.27452 30.94952) (width 0.2) (layer "F.Cu") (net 11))
 (segment (start 67.81952 35.06952) (end 71.68048 35.06952) (width 0.2) (layer "F.Cu") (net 11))
 (segment (start 74.27452 30.94952) (end 73.5 30.175) (width 0.2) (layer "F.Cu") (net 11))
 (segment (start 73.35 30.025) (end 73.35 27.25) (width 0.25) (layer "F.Cu") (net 11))
 (segment (start 66.05 33.795) (end 66.545 33.795) (width 0.2) (layer "F.Cu") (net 11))
 (segment (start 66.545 33.795) (end 67.81952 35.06952) (width 0.2) (layer "F.Cu") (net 11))
 (segment (start 62.95 30) (end 61.825 30) (width 0.508) (layer "F.Cu") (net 1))
 (segment (start 61.825 30) (end 61.325 30.5) (width 0.508) (layer "F.Cu") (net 1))
 (via (at 59.5 32.5) (size 0.8) (drill 0.4) (layers "F.Cu" "B.Cu") (free) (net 1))
 (via (at 64.5 34.5) (size 0.8) (drill 0.4) (layers "F.Cu" "B.Cu") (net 1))
 (via (at 61.75 31.5) (size 0.8) (drill 0.4) (layers "F.Cu" "B.Cu") (free) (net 1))
 (via (at 67.25 33) (size 0.8) (drill 0.4) (layers "F.Cu" "B.Cu") (free) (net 1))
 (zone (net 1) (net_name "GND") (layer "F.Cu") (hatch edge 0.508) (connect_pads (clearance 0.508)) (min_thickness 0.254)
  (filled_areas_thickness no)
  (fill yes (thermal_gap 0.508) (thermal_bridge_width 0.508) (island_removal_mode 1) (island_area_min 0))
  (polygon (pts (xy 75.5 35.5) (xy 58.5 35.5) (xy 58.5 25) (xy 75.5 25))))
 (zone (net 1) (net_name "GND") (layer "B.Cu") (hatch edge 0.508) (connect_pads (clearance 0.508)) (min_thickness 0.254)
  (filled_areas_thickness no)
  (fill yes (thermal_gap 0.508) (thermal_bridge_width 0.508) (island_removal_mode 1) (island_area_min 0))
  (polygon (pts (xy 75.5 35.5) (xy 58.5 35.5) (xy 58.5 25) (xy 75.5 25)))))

